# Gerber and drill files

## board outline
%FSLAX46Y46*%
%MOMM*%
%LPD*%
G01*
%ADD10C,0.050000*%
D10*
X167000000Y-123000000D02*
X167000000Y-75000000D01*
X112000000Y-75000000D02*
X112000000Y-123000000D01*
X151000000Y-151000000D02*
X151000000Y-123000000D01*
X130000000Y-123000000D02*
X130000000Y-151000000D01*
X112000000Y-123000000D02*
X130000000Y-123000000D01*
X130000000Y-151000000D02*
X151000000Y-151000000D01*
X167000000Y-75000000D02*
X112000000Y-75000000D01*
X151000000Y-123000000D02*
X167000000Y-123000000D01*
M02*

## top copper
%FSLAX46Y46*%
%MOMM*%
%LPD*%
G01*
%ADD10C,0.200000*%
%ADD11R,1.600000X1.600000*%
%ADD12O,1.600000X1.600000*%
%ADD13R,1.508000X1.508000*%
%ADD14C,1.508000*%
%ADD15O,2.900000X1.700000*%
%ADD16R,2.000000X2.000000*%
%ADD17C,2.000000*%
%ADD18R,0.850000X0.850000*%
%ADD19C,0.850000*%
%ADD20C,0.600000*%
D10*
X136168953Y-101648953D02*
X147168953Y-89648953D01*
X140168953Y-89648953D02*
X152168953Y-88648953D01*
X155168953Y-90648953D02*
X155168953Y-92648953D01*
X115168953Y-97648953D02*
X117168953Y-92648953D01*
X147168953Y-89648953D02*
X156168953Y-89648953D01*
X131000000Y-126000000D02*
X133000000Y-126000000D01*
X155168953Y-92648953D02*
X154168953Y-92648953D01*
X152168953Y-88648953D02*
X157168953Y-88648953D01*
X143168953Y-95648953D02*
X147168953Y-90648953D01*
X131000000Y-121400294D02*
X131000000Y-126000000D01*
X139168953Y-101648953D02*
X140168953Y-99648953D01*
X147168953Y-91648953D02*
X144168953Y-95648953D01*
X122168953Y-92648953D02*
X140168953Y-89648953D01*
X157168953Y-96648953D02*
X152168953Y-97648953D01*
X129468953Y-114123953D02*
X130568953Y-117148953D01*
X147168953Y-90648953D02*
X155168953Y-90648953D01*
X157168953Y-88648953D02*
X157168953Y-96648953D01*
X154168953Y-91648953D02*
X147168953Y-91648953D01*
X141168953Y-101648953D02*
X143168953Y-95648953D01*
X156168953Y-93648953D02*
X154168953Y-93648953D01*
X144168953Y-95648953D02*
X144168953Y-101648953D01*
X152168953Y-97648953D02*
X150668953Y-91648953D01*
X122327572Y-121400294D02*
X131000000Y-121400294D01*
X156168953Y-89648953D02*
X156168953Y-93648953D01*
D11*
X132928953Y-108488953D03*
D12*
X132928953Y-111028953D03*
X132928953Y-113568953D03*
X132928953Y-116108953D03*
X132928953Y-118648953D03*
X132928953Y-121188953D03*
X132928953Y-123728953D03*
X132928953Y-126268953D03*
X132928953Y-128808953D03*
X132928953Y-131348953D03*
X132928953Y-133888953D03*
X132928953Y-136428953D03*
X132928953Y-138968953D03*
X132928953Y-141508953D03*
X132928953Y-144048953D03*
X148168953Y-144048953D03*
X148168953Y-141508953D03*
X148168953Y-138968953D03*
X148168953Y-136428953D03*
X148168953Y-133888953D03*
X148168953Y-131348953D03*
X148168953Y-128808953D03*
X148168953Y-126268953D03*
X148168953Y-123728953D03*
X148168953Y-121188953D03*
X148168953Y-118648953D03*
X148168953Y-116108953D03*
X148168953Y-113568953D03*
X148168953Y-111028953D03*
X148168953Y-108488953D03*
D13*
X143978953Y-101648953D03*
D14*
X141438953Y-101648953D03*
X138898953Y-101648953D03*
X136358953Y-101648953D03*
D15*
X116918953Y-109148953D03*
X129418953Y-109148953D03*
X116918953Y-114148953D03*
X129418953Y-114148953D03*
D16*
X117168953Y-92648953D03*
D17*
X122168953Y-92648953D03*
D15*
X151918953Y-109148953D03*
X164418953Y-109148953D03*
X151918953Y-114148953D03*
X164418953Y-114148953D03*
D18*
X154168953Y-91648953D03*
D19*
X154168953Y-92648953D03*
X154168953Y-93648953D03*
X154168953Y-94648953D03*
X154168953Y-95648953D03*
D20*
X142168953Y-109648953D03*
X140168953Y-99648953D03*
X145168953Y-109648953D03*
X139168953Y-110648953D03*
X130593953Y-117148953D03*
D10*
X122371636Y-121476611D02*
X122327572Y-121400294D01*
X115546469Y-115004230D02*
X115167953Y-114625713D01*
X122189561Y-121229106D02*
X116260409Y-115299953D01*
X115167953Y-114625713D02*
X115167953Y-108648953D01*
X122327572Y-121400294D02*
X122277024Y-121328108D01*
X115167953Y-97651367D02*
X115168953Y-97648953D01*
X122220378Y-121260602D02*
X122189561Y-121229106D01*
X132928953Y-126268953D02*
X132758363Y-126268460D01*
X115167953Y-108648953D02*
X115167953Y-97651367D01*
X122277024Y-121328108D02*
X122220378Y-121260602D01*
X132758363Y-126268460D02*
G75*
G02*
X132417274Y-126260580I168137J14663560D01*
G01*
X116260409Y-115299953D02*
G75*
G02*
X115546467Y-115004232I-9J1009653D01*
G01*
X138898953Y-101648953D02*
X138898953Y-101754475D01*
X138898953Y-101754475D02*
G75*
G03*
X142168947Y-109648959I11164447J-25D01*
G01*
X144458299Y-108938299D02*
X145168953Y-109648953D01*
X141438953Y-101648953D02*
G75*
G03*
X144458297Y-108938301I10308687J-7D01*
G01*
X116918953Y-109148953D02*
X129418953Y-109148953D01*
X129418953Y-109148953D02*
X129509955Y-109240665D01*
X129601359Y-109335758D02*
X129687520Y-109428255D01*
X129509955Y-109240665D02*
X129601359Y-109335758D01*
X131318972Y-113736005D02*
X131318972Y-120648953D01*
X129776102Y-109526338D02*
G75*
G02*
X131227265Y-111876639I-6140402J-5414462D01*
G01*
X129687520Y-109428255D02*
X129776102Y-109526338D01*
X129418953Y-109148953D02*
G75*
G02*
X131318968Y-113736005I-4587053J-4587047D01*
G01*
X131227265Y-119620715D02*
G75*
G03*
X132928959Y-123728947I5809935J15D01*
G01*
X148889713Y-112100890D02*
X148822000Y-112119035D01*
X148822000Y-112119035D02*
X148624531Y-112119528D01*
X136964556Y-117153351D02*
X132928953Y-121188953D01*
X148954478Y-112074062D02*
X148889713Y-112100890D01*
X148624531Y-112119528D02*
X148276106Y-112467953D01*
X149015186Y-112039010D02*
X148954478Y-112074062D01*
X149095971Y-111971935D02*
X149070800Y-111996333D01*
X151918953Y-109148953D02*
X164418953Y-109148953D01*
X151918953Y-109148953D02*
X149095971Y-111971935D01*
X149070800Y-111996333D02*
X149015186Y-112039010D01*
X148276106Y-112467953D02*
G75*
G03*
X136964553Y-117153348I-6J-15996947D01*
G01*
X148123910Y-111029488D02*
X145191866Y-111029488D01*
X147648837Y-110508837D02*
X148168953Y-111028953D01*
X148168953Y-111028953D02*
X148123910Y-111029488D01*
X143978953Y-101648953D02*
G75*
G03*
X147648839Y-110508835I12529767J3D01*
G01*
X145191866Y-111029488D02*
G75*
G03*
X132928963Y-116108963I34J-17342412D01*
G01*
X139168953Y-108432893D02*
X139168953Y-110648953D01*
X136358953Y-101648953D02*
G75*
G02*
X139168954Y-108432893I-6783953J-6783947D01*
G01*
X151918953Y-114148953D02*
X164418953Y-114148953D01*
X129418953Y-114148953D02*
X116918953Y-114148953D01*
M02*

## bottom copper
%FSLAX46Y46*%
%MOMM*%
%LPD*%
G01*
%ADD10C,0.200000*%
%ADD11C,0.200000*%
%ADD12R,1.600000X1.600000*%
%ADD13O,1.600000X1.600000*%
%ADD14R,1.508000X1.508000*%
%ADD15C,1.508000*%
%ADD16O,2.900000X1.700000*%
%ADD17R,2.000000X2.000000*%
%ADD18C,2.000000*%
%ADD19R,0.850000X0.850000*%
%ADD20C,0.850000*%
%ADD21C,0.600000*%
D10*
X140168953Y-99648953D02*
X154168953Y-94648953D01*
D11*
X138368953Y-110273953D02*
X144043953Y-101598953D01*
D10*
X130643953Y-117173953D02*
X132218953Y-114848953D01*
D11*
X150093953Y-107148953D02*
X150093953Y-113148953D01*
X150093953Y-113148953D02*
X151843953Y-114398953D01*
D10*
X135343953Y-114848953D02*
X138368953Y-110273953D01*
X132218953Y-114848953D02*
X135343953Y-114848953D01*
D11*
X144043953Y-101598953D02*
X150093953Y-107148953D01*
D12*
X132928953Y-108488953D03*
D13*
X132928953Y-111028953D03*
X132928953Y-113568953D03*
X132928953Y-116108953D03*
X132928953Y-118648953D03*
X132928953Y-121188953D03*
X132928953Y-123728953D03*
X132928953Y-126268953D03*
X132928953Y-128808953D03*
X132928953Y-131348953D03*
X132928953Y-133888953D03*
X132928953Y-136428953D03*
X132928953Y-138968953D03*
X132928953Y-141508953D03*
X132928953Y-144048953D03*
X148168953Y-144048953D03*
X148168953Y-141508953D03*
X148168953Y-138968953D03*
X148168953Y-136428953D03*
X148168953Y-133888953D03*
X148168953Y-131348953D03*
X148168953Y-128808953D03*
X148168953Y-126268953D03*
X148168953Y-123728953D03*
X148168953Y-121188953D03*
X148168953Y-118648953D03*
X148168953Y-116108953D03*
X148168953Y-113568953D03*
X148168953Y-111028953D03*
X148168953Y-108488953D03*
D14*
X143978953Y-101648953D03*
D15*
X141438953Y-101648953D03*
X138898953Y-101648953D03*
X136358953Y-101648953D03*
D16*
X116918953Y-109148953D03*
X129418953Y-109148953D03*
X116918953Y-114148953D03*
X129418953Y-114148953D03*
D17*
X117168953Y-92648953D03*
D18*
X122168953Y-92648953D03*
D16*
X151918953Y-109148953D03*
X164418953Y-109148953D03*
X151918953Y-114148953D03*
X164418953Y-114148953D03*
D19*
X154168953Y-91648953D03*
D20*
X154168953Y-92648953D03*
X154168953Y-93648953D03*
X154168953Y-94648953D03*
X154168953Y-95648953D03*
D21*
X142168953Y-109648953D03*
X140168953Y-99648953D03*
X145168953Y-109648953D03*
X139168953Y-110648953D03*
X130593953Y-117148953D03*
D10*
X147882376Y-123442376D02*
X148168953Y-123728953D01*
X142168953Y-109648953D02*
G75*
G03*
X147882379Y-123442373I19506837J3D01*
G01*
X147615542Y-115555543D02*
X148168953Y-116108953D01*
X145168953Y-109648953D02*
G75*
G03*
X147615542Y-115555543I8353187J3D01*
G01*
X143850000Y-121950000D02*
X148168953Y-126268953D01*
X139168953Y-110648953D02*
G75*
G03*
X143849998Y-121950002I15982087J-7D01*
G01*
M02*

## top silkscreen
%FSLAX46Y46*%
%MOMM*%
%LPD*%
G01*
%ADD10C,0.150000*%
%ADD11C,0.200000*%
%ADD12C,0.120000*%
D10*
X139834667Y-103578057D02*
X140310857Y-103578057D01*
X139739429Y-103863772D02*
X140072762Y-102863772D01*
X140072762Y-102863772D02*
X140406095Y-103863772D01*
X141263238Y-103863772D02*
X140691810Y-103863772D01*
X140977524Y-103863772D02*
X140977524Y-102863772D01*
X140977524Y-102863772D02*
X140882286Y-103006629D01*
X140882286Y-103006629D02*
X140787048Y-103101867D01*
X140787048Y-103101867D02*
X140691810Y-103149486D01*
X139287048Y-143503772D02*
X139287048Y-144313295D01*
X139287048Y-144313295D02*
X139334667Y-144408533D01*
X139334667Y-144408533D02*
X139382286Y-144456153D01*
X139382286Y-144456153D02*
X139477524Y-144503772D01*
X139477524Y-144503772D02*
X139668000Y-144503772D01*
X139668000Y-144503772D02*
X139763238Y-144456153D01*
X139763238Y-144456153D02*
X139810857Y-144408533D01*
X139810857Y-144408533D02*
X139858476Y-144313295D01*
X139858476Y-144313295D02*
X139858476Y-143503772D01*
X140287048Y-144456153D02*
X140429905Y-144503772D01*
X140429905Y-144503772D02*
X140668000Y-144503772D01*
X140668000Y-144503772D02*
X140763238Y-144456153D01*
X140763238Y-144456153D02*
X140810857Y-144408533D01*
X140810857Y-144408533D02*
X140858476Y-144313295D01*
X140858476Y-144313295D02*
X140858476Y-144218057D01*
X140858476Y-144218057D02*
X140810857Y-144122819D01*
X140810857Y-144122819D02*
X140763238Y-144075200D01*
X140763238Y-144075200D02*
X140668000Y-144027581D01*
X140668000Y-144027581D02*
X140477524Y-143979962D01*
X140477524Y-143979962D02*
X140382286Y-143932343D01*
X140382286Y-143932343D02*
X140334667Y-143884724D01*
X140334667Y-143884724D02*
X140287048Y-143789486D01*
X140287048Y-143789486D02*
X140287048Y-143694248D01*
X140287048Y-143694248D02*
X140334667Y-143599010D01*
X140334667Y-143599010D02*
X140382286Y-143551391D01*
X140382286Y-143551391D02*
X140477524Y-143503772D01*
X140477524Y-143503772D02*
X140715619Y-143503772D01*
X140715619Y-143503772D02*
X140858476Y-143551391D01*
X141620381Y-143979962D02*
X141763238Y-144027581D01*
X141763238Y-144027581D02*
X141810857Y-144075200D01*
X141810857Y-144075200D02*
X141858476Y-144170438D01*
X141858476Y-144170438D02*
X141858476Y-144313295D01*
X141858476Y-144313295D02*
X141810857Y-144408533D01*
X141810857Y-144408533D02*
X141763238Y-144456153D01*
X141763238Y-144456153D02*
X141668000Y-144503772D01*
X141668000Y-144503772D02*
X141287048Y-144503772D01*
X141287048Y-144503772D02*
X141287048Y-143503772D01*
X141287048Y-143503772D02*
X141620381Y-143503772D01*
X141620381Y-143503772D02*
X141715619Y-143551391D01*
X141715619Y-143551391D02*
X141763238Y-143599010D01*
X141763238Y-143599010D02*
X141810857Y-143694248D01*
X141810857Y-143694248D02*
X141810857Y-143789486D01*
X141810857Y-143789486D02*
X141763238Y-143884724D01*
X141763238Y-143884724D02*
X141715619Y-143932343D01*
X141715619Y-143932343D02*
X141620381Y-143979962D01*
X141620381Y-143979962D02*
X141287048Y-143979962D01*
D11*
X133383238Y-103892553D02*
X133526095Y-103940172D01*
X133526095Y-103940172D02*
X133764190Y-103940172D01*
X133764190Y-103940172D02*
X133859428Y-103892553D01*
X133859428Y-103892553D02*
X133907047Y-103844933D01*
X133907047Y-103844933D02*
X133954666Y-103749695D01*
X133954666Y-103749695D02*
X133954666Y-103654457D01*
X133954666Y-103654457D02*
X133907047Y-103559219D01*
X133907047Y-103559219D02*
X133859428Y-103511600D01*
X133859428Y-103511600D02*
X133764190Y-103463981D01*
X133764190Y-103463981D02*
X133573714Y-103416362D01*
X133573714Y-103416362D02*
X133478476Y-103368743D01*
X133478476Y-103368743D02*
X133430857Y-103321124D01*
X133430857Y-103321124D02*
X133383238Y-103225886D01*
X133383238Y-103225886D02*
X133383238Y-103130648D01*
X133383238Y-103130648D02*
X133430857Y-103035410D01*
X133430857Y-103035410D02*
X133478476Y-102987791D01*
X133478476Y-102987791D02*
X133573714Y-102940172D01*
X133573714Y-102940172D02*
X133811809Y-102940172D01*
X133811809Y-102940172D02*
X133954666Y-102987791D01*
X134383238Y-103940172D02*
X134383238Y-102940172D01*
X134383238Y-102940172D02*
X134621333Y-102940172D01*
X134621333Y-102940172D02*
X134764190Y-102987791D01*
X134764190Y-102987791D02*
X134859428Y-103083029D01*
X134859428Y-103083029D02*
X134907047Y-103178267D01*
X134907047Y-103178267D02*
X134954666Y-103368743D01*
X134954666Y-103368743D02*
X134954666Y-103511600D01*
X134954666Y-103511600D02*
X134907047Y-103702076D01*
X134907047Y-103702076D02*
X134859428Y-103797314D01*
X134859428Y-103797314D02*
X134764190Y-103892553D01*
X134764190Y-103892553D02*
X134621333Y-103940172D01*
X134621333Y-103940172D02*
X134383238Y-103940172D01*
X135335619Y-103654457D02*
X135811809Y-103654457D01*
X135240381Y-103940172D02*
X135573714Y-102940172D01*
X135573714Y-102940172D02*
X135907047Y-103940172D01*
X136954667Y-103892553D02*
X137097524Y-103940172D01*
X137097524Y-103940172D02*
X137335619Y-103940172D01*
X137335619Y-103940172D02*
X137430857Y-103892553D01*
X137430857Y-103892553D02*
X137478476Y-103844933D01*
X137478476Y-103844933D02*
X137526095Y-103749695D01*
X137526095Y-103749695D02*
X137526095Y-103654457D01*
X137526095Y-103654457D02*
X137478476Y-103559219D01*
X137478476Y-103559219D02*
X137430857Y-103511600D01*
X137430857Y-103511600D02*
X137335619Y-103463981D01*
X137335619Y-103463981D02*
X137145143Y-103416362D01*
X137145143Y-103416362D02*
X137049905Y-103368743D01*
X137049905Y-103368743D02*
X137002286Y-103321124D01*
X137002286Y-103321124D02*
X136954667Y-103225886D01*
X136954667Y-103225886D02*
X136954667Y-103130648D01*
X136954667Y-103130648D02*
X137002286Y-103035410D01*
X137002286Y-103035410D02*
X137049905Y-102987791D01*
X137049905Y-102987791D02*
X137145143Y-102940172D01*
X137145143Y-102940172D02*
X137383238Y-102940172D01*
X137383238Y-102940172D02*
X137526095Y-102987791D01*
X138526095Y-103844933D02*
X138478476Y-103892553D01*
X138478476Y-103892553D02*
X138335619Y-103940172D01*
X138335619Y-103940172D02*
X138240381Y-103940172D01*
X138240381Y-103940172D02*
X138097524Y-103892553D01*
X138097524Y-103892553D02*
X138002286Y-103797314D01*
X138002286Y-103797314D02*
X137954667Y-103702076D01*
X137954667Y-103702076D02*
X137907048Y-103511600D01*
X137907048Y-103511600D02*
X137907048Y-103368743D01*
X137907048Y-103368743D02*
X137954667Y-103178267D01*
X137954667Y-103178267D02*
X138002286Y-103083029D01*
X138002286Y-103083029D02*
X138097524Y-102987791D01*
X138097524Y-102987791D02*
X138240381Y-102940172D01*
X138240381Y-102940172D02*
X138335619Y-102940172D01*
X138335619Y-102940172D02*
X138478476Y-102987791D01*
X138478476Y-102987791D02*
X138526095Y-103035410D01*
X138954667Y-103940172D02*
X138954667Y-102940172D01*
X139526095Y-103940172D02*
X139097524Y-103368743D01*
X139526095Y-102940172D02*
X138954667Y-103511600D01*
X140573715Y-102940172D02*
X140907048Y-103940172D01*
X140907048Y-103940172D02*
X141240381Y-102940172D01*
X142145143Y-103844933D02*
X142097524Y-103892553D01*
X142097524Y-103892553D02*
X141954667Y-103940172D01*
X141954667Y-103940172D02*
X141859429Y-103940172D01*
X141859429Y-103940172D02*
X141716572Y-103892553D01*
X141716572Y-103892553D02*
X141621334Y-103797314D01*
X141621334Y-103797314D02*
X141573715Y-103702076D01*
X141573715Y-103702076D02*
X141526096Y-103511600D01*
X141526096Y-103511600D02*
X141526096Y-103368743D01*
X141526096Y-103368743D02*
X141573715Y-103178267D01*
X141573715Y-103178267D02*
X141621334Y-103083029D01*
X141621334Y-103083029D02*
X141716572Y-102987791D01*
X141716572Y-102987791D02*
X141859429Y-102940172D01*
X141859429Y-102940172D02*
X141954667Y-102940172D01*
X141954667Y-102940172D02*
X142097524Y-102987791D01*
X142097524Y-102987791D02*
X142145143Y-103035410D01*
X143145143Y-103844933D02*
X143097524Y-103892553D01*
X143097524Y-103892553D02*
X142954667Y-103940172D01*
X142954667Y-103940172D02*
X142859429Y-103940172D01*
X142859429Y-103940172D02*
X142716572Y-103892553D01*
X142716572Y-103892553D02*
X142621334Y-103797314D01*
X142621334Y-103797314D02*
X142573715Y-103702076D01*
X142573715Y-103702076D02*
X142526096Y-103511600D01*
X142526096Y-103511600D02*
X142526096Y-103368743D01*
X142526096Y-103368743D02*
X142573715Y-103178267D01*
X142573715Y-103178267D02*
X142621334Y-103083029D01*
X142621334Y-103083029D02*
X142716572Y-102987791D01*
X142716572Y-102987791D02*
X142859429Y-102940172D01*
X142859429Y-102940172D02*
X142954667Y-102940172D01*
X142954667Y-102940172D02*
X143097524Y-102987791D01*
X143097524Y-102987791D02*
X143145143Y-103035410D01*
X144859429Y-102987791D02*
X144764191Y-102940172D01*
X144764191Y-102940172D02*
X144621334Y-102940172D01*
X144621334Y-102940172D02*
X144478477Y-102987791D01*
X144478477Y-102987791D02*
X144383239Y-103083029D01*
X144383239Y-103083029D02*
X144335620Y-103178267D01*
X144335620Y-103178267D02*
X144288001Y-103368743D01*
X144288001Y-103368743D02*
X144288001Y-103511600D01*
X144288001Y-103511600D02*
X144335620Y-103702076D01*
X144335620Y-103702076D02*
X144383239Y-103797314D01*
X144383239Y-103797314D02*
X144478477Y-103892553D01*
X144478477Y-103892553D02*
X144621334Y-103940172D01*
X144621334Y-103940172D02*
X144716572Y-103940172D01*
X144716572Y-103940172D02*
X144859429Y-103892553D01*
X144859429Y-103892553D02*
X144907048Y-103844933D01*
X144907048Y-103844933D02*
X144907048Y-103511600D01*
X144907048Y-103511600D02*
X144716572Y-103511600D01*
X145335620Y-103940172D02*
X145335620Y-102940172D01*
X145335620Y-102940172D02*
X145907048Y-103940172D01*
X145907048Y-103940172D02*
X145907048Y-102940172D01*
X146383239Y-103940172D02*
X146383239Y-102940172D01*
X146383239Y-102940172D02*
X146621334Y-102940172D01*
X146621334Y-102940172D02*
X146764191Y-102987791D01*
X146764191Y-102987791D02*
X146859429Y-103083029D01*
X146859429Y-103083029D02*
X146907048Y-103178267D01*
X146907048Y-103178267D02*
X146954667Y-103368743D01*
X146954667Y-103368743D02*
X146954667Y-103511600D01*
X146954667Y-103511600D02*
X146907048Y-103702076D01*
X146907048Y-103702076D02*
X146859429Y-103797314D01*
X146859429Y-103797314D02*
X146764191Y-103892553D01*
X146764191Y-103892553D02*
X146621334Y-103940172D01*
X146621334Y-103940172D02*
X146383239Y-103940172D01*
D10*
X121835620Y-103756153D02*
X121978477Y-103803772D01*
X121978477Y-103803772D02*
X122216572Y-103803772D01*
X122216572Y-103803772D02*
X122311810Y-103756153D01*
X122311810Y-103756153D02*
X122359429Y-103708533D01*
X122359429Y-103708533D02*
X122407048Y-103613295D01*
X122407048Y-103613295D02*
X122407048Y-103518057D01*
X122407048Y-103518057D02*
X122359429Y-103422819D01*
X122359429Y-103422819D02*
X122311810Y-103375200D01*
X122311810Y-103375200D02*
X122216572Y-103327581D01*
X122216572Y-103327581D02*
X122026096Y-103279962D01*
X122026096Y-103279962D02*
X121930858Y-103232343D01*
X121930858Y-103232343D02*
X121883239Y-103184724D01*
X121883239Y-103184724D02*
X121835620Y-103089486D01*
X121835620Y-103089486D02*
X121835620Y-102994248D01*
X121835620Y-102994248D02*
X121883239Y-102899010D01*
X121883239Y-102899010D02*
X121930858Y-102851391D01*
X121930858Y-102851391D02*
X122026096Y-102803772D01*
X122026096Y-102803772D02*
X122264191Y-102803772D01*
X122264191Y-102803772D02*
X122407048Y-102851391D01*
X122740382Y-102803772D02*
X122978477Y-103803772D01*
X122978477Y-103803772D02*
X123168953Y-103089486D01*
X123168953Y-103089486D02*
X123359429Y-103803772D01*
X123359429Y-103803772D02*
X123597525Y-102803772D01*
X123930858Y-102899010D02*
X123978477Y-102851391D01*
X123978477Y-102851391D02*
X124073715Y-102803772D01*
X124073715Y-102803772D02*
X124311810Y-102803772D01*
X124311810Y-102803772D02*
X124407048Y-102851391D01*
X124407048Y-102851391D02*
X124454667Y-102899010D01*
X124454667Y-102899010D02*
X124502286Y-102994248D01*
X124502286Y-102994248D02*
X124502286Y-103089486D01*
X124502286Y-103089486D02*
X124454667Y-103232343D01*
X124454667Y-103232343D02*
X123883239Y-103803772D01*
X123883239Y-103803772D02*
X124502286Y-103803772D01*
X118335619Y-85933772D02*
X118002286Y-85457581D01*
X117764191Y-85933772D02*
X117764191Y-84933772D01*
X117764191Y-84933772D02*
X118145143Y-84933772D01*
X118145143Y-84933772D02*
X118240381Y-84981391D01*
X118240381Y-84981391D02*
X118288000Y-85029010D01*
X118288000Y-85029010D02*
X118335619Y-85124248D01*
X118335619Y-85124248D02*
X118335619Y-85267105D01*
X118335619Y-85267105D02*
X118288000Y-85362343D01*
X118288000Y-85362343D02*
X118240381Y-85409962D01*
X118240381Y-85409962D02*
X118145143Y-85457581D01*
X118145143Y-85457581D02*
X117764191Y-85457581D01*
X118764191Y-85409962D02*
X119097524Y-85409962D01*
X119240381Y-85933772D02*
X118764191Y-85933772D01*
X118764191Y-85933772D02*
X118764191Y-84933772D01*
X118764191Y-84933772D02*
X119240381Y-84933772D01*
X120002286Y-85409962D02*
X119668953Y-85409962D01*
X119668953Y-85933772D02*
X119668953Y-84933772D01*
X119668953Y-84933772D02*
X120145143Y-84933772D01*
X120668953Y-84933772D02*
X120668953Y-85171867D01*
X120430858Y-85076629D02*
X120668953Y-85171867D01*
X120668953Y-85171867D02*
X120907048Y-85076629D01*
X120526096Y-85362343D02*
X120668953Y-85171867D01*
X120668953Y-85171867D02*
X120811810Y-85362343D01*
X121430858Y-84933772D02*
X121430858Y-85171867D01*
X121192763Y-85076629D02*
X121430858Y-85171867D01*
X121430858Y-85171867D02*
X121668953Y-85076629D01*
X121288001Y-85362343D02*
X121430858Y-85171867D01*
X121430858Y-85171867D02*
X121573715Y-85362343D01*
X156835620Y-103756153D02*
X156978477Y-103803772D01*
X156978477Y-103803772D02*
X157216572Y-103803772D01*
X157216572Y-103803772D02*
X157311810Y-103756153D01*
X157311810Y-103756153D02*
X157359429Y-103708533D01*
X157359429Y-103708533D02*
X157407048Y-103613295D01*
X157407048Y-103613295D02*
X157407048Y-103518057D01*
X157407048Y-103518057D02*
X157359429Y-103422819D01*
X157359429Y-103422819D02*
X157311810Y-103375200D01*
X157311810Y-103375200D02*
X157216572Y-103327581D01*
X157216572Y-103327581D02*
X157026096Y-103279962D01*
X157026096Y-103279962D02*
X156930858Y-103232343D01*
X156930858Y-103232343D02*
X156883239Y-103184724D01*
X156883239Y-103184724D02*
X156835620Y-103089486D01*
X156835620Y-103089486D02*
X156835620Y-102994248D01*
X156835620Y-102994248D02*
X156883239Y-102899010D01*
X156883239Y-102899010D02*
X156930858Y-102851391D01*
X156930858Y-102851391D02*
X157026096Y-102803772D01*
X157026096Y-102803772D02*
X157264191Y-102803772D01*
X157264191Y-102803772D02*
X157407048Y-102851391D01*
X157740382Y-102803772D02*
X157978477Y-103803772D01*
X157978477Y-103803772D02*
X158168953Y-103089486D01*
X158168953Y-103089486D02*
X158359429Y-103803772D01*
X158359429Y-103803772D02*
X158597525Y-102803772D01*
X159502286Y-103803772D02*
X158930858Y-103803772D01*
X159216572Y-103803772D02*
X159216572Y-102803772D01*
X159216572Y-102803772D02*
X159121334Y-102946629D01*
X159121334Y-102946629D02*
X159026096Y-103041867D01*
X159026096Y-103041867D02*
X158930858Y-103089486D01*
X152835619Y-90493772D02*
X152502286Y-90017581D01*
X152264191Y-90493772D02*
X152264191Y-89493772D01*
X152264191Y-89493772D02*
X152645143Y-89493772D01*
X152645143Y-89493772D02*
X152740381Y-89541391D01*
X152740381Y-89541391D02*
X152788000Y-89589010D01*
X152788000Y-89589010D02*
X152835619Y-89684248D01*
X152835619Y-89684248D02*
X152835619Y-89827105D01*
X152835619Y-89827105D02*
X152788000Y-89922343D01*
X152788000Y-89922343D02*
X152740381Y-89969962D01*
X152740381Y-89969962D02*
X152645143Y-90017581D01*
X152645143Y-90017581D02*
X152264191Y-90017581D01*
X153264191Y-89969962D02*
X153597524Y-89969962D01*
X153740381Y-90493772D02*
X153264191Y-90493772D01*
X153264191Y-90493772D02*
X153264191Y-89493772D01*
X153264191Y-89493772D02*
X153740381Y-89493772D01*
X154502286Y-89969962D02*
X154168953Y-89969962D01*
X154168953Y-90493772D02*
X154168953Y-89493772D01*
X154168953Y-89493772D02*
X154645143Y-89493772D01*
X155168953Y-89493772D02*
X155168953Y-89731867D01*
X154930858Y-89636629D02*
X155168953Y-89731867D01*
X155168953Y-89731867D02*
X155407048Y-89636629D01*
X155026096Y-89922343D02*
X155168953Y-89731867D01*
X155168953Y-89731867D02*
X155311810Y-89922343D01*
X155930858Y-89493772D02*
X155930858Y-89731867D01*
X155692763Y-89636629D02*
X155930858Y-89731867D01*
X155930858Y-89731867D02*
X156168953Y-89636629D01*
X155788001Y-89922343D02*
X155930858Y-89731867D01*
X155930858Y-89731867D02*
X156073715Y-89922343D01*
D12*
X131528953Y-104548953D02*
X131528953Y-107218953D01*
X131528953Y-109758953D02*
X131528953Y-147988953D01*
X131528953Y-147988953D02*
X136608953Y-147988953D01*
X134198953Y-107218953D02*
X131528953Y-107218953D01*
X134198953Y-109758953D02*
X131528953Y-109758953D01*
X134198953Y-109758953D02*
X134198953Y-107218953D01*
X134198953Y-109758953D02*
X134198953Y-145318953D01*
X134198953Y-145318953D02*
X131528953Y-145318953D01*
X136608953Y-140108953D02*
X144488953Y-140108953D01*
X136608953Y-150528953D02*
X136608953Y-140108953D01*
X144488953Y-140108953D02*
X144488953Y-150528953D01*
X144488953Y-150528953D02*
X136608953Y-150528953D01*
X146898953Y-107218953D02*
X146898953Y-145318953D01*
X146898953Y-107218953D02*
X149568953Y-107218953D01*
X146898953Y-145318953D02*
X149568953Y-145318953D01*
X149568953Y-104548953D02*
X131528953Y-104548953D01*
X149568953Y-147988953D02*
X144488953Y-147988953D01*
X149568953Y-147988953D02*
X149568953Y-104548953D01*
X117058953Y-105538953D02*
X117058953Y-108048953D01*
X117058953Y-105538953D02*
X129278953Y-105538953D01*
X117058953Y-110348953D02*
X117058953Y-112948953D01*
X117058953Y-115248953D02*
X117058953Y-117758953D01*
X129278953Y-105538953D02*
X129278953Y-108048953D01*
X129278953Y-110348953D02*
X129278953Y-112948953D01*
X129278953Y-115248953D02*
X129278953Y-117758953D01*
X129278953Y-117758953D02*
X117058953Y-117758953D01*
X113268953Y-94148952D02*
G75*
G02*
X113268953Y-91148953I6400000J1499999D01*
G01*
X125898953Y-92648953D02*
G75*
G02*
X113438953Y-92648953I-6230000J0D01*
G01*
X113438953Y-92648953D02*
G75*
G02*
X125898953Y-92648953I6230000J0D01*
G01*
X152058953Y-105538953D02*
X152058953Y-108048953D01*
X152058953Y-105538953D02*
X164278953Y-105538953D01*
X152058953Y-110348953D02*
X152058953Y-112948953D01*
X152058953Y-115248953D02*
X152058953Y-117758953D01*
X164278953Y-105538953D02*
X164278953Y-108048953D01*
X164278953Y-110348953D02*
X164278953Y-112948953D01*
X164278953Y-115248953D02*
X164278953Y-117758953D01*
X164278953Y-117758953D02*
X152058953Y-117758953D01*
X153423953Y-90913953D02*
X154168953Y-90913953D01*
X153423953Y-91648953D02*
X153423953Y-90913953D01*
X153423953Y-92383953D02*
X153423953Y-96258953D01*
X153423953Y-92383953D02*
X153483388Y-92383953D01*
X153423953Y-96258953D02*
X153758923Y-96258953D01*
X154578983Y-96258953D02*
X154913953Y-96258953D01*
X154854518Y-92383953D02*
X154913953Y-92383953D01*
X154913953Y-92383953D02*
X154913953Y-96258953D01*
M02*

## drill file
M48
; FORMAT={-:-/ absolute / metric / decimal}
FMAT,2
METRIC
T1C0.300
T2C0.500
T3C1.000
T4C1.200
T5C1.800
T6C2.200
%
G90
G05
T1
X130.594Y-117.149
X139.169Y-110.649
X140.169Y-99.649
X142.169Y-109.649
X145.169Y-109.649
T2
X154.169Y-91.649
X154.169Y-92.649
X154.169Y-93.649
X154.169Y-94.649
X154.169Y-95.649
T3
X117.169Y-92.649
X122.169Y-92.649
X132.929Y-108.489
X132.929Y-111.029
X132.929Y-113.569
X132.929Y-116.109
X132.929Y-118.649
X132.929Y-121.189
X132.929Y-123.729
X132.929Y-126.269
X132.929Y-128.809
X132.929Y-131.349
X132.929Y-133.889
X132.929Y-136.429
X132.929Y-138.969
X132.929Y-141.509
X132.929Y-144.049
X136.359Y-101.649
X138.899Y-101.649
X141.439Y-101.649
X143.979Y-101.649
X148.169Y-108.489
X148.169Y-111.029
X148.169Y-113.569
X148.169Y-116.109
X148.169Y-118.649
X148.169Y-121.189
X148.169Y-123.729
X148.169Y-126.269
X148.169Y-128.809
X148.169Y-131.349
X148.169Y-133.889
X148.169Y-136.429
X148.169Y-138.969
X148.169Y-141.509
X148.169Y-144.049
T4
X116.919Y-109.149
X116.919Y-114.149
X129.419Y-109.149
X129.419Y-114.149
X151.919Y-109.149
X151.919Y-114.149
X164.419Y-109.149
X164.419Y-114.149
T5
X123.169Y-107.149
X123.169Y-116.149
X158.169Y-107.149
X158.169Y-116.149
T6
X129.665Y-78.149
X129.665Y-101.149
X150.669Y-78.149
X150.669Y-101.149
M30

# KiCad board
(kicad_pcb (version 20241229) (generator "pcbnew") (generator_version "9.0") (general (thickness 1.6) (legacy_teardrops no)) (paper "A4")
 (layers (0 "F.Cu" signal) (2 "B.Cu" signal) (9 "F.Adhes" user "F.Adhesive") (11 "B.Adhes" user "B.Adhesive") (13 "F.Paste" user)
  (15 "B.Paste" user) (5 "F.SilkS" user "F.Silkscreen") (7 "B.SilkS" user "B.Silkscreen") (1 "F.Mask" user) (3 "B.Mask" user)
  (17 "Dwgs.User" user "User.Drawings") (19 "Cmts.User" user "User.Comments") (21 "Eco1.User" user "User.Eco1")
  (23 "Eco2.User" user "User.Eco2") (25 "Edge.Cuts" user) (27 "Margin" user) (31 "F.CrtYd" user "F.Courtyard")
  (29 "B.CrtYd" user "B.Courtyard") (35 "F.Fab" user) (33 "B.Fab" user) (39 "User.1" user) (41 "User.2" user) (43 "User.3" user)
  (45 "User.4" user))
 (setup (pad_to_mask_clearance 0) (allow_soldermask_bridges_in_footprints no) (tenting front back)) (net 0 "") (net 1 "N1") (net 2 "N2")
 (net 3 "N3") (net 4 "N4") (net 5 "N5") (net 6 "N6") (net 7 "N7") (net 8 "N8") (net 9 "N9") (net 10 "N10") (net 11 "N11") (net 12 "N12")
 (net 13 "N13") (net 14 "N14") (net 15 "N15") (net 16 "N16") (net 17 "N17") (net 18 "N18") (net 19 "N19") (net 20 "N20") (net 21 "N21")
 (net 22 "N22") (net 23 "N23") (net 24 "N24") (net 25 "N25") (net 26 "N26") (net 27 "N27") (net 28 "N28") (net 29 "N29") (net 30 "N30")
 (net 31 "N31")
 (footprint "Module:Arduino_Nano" (layer "F.Cu") (at 132.928953 108.488953)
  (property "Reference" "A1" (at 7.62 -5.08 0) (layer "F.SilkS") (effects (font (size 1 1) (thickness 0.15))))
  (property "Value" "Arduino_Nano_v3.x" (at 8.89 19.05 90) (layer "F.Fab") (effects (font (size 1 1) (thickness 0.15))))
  (fp_line (start -1.4 -3.94) (end -1.4 -1.27) (stroke (width 0.12) (type solid)) (layer "F.SilkS"))
  (fp_line (start -1.4 1.27) (end -1.4 39.5) (stroke (width 0.12) (type solid)) (layer "F.SilkS"))
  (fp_line (start -1.4 39.5) (end 3.68 39.5) (stroke (width 0.12) (type solid)) (layer "F.SilkS"))
  (fp_line (start 1.27 -1.27) (end -1.4 -1.27) (stroke (width 0.12) (type solid)) (layer "F.SilkS"))
  (fp_line (start 1.27 1.27) (end -1.4 1.27) (stroke (width 0.12) (type solid)) (layer "F.SilkS"))
  (fp_line (start 1.27 1.27) (end 1.27 -1.27) (stroke (width 0.12) (type solid)) (layer "F.SilkS"))
  (fp_line (start 1.27 1.27) (end 1.27 36.83) (stroke (width 0.12) (type solid)) (layer "F.SilkS"))
  (fp_line (start 1.27 36.83) (end -1.4 36.83) (stroke (width 0.12) (type solid)) (layer "F.SilkS"))
  (fp_line (start 3.68 31.62) (end 11.56 31.62) (stroke (width 0.12) (type solid)) (layer "F.SilkS"))
  (fp_line (start 3.68 42.04) (end 3.68 31.62) (stroke (width 0.12) (type solid)) (layer "F.SilkS"))
  (fp_line (start 11.56 31.62) (end 11.56 42.04) (stroke (width 0.12) (type solid)) (layer "F.SilkS"))
  (fp_line (start 11.56 42.04) (end 3.68 42.04) (stroke (width 0.12) (type solid)) (layer "F.SilkS"))
  (fp_line (start 13.97 -1.27) (end 13.97 36.83) (stroke (width 0.12) (type solid)) (layer "F.SilkS"))
  (fp_line (start 13.97 -1.27) (end 16.64 -1.27) (stroke (width 0.12) (type solid)) (layer "F.SilkS"))
  (fp_line (start 13.97 36.83) (end 16.64 36.83) (stroke (width 0.12) (type solid)) (layer "F.SilkS"))
  (fp_line (start 16.64 -3.94) (end -1.4 -3.94) (stroke (width 0.12) (type solid)) (layer "F.SilkS"))
  (fp_line (start 16.64 39.5) (end 11.56 39.5) (stroke (width 0.12) (type solid)) (layer "F.SilkS"))
  (fp_line (start 16.64 39.5) (end 16.64 -3.94) (stroke (width 0.12) (type solid)) (layer "F.SilkS"))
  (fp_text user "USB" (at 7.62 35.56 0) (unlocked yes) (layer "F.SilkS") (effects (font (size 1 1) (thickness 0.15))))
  (pad "1" thru_hole rect (at 0 0) (size 1.6 1.6) (drill 1) (layers "*.Cu" "*.Mask") (remove_unused_layers no) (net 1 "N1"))
  (pad "2" thru_hole oval (at 0 2.54) (size 1.6 1.6) (drill 1) (layers "*.Cu" "*.Mask") (remove_unused_layers no) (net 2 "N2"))
  (pad "3" thru_hole oval (at 0 5.08) (size 1.6 1.6) (drill 1) (layers "*.Cu" "*.Mask") (remove_unused_layers no) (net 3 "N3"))
  (pad "4" thru_hole oval (at 0 7.62) (size 1.6 1.6) (drill 1) (layers "*.Cu" "*.Mask") (remove_unused_layers no) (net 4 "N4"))
  (pad "5" thru_hole oval (at 0 10.16) (size 1.6 1.6) (drill 1) (layers "*.Cu" "*.Mask") (remove_unused_layers no) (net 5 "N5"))
  (pad "6" thru_hole oval (at 0 12.7) (size 1.6 1.6) (drill 1) (layers "*.Cu" "*.Mask") (remove_unused_layers no) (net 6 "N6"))
  (pad "7" thru_hole oval (at 0 15.24) (size 1.6 1.6) (drill 1) (layers "*.Cu" "*.Mask") (remove_unused_layers no) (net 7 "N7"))
  (pad "8" thru_hole oval (at 0 17.78) (size 1.6 1.6) (drill 1) (layers "*.Cu" "*.Mask") (remove_unused_layers no) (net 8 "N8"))
  (pad "9" thru_hole oval (at 0 20.32) (size 1.6 1.6) (drill 1) (layers "*.Cu" "*.Mask") (remove_unused_layers no) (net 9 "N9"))
  (pad "10" thru_hole oval (at 0 22.86) (size 1.6 1.6) (drill 1) (layers "*.Cu" "*.Mask") (remove_unused_layers no) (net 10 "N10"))
  (pad "11" thru_hole oval (at 0 25.4) (size 1.6 1.6) (drill 1) (layers "*.Cu" "*.Mask") (remove_unused_layers no) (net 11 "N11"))
  (pad "12" thru_hole oval (at 0 27.94) (size 1.6 1.6) (drill 1) (layers "*.Cu" "*.Mask") (remove_unused_layers no) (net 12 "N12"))
  (pad "13" thru_hole oval (at 0 30.48) (size 1.6 1.6) (drill 1) (layers "*.Cu" "*.Mask") (remove_unused_layers no) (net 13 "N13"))
  (pad "14" thru_hole oval (at 0 33.02) (size 1.6 1.6) (drill 1) (layers "*.Cu" "*.Mask") (remove_unused_layers no) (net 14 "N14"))
  (pad "15" thru_hole oval (at 0 35.56) (size 1.6 1.6) (drill 1) (layers "*.Cu" "*.Mask") (remove_unused_layers no) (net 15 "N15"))
  (pad "16" thru_hole oval (at 15.24 35.56) (size 1.6 1.6) (drill 1) (layers "*.Cu" "*.Mask") (remove_unused_layers no) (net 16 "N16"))
  (pad "17" thru_hole oval (at 15.24 33.02) (size 1.6 1.6) (drill 1) (layers "*.Cu" "*.Mask") (remove_unused_layers no) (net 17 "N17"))
  (pad "18" thru_hole oval (at 15.24 30.48) (size 1.6 1.6) (drill 1) (layers "*.Cu" "*.Mask") (remove_unused_layers no) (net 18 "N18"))
  (pad "19" thru_hole oval (at 15.24 27.94) (size 1.6 1.6) (drill 1) (layers "*.Cu" "*.Mask") (remove_unused_layers no) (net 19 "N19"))
  (pad "20" thru_hole oval (at 15.24 25.4) (size 1.6 1.6) (drill 1) (layers "*.Cu" "*.Mask") (remove_unused_layers no) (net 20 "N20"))
  (pad "21" thru_hole oval (at 15.24 22.86) (size 1.6 1.6) (drill 1) (layers "*.Cu" "*.Mask") (remove_unused_layers no) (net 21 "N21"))
  (pad "22" thru_hole oval (at 15.24 20.32) (size 1.6 1.6) (drill 1) (layers "*.Cu" "*.Mask") (remove_unused_layers no) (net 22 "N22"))
  (pad "23" thru_hole oval (at 15.24 17.78) (size 1.6 1.6) (drill 1) (layers "*.Cu" "*.Mask") (remove_unused_layers no) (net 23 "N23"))
  (pad "24" thru_hole oval (at 15.24 15.24) (size 1.6 1.6) (drill 1) (layers "*.Cu" "*.Mask") (remove_unused_layers no) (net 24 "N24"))
  (pad "25" thru_hole oval (at 15.24 12.7) (size 1.6 1.6) (drill 1) (layers "*.Cu" "*.Mask") (remove_unused_layers no) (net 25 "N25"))
  (pad "26" thru_hole oval (at 15.24 10.16) (size 1.6 1.6) (drill 1) (layers "*.Cu" "*.Mask") (remove_unused_layers no) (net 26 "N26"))
  (pad "27" thru_hole oval (at 15.24 7.62) (size 1.6 1.6) (drill 1) (layers "*.Cu" "*.Mask") (remove_unused_layers no) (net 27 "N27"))
  (pad "28" thru_hole oval (at 15.24 5.08) (size 1.6 1.6) (drill 1) (layers "*.Cu" "*.Mask") (remove_unused_layers no) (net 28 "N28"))
  (pad "29" thru_hole oval (at 15.24 2.54) (size 1.6 1.6) (drill 1) (layers "*.Cu" "*.Mask") (remove_unused_layers no) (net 4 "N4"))
  (pad "30" thru_hole oval (at 15.24 0) (size 1.6 1.6) (drill 1) (layers "*.Cu" "*.Mask") (remove_unused_layers no) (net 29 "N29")))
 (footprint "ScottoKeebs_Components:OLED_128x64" (layer "F.Cu") (at 140.168953 89.648953)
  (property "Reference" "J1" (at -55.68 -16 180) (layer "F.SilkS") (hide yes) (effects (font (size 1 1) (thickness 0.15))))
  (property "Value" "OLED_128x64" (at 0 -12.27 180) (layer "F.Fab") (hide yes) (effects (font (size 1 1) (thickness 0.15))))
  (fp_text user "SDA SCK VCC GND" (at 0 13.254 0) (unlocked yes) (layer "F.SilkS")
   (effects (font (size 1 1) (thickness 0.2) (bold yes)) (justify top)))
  (pad "" np_thru_hole circle (at -10.50445 -11.5 180) (size 2.2 2.2) (drill 2.2) (layers "*.Cu" "*.Mask") (solder_mask_margin 0.102))
  (pad "" np_thru_hole circle (at -10.50445 11.5 180) (size 2.2 2.2) (drill 2.2) (layers "*.Cu" "*.Mask") (solder_mask_margin 0.102))
  (pad "" np_thru_hole circle (at 10.5 -11.5 180) (size 2.2 2.2) (drill 2.2) (layers "*.Cu" "*.Mask") (solder_mask_margin 0.102))
  (pad "" np_thru_hole circle (at 10.5 11.5 180) (size 2.2 2.2) (drill 2.2) (layers "*.Cu" "*.Mask") (solder_mask_margin 0.102))
  (pad "1" thru_hole rect (at 3.81 12 180) (size 1.508 1.508) (drill 1) (layers "*.Cu" "*.Mask") (remove_unused_layers no) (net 4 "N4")
   (solder_mask_margin 0.102))
  (pad "2" thru_hole circle (at 1.27 12 180) (size 1.508 1.508) (drill 1) (layers "*.Cu" "*.Mask") (remove_unused_layers no) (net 27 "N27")
   (solder_mask_margin 0.102))
  (pad "3" thru_hole circle (at -1.27 12 180) (size 1.508 1.508) (drill 1) (layers "*.Cu" "*.Mask") (remove_unused_layers no) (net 24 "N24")
   (solder_mask_margin 0.102))
  (pad "4" thru_hole circle (at -3.81 12 180) (size 1.508 1.508) (drill 1) (layers "*.Cu" "*.Mask") (remove_unused_layers no) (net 23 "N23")
   (solder_mask_margin 0.102)))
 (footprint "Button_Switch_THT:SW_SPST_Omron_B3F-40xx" (layer "F.Cu") (at 116.918953 109.148953)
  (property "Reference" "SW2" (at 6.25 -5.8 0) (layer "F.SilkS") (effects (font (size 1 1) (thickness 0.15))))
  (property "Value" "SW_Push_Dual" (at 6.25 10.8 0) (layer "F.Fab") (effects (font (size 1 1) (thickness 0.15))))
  (fp_line (start 0.14 -3.61) (end 0.14 -1.1) (stroke (width 0.12) (type default)) (layer "F.SilkS"))
  (fp_line (start 0.14 -3.61) (end 12.36 -3.61) (stroke (width 0.12) (type default)) (layer "F.SilkS"))
  (fp_line (start 0.14 1.2) (end 0.14 3.8) (stroke (width 0.12) (type default)) (layer "F.SilkS"))
  (fp_line (start 0.14 6.1) (end 0.14 8.61) (stroke (width 0.12) (type default)) (layer "F.SilkS"))
  (fp_line (start 12.36 -3.61) (end 12.36 -1.1) (stroke (width 0.12) (type default)) (layer "F.SilkS"))
  (fp_line (start 12.36 1.2) (end 12.36 3.8) (stroke (width 0.12) (type default)) (layer "F.SilkS"))
  (fp_line (start 12.36 6.1) (end 12.36 8.61) (stroke (width 0.12) (type default)) (layer "F.SilkS"))
  (fp_line (start 12.36 8.61) (end 0.14 8.61) (stroke (width 0.12) (type default)) (layer "F.SilkS"))
  (pad "" np_thru_hole circle (at 6.25 -2) (size 1.8 1.8) (drill 1.8) (layers "*.Cu" "*.Mask"))
  (pad "" np_thru_hole circle (at 6.25 7) (size 1.8 1.8) (drill 1.8) (layers "*.Cu" "*.Mask"))
  (pad "1" thru_hole oval (at 0 0) (size 2.9 1.7) (drill 1.2) (layers "*.Cu" "*.Mask") (remove_unused_layers no) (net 7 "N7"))
  (pad "1" thru_hole oval (at 12.5 0) (size 2.9 1.7) (drill 1.2) (layers "*.Cu" "*.Mask") (remove_unused_layers no) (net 7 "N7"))
  (pad "2" thru_hole oval (at 0 5) (size 2.9 1.7) (drill 1.2) (layers "*.Cu" "*.Mask") (remove_unused_layers no) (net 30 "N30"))
  (pad "2" thru_hole oval (at 12.5 5) (size 2.9 1.7) (drill 1.2) (layers "*.Cu" "*.Mask") (remove_unused_layers no) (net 30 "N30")))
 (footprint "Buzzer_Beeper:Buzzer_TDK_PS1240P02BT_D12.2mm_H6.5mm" (layer "F.Cu") (at 117.168953 92.648953)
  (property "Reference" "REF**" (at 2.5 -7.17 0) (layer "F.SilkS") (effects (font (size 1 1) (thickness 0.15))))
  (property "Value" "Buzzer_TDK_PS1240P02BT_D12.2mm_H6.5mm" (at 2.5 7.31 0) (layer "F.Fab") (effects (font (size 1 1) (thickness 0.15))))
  (fp_arc (start -3.9 1.499999) (mid -4.073431 0) (end -3.9 -1.5) (stroke (width 0.12) (type solid)) (layer "F.SilkS"))
  (fp_circle (center 2.5 0) (end 8.73 0) (stroke (width 0.12) (type solid)) (fill no) (layer "F.SilkS"))
  (pad "1" thru_hole rect (at 0 0) (size 2 2) (drill 1) (layers "*.Cu" "*.Mask") (remove_unused_layers no))
  (pad "2" thru_hole circle (at 5 0) (size 2 2) (drill 1) (layers "*.Cu" "*.Mask") (remove_unused_layers no)))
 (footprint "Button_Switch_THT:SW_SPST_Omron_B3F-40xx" (layer "F.Cu") (at 151.918953 109.148953)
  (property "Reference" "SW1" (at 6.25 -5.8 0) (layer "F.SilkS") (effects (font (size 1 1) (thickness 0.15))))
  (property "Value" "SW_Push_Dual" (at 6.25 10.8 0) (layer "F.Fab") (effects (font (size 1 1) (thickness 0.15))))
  (fp_line (start 0.14 -3.61) (end 0.14 -1.1) (stroke (width 0.12) (type default)) (layer "F.SilkS"))
  (fp_line (start 0.14 -3.61) (end 12.36 -3.61) (stroke (width 0.12) (type default)) (layer "F.SilkS"))
  (fp_line (start 0.14 1.2) (end 0.14 3.8) (stroke (width 0.12) (type default)) (layer "F.SilkS"))
  (fp_line (start 0.14 6.1) (end 0.14 8.61) (stroke (width 0.12) (type default)) (layer "F.SilkS"))
  (fp_line (start 12.36 -3.61) (end 12.36 -1.1) (stroke (width 0.12) (type default)) (layer "F.SilkS"))
  (fp_line (start 12.36 1.2) (end 12.36 3.8) (stroke (width 0.12) (type default)) (layer "F.SilkS"))
  (fp_line (start 12.36 6.1) (end 12.36 8.61) (stroke (width 0.12) (type default)) (layer "F.SilkS"))
  (fp_line (start 12.36 8.61) (end 0.14 8.61) (stroke (width 0.12) (type default)) (layer "F.SilkS"))
  (pad "" np_thru_hole circle (at 6.25 -2) (size 1.8 1.8) (drill 1.8) (layers "*.Cu" "*.Mask"))
  (pad "" np_thru_hole circle (at 6.25 7) (size 1.8 1.8) (drill 1.8) (layers "*.Cu" "*.Mask"))
  (pad "1" thru_hole oval (at 0 0) (size 2.9 1.7) (drill 1.2) (layers "*.Cu" "*.Mask") (remove_unused_layers no) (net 6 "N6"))
  (pad "1" thru_hole oval (at 12.5 0) (size 2.9 1.7) (drill 1.2) (layers "*.Cu" "*.Mask") (remove_unused_layers no) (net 6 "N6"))
  (pad "2" thru_hole oval (at 0 5) (size 2.9 1.7) (drill 1.2) (layers "*.Cu" "*.Mask") (remove_unused_layers no) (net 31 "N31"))
  (pad "2" thru_hole oval (at 12.5 5) (size 2.9 1.7) (drill 1.2) (layers "*.Cu" "*.Mask") (remove_unused_layers no) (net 31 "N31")))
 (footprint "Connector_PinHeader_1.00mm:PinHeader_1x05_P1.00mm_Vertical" (layer "F.Cu") (at 154.168953 91.648953)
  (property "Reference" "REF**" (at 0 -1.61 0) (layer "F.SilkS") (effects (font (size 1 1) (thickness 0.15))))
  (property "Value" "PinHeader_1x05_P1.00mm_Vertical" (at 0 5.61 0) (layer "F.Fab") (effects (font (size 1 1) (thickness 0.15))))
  (fp_line (start -0.745 -0.735) (end 0 -0.735) (stroke (width 0.12) (type solid)) (layer "F.SilkS"))
  (fp_line (start -0.745 0) (end -0.745 -0.735) (stroke (width 0.12) (type solid)) (layer "F.SilkS"))
  (fp_line (start -0.745 0.735) (end -0.745 4.61) (stroke (width 0.12) (type solid)) (layer "F.SilkS"))
  (fp_line (start -0.745 0.735) (end -0.685565 0.735) (stroke (width 0.12) (type solid)) (layer "F.SilkS"))
  (fp_line (start -0.745 4.61) (end -0.41003 4.61) (stroke (width 0.12) (type solid)) (layer "F.SilkS"))
  (fp_line (start 0.41003 4.61) (end 0.745 4.61) (stroke (width 0.12) (type solid)) (layer "F.SilkS"))
  (fp_line (start 0.685565 0.735) (end 0.745 0.735) (stroke (width 0.12) (type solid)) (layer "F.SilkS"))
  (fp_line (start 0.745 0.735) (end 0.745 4.61) (stroke (width 0.12) (type solid)) (layer "F.SilkS"))
  (pad "1" thru_hole rect (at 0 0) (size 0.85 0.85) (drill 0.5) (layers "*.Cu" "*.Mask") (remove_unused_layers no))
  (pad "2" thru_hole circle (at 0 1) (size 0.85 0.85) (drill 0.5) (layers "*.Cu" "*.Mask") (remove_unused_layers no))
  (pad "3" thru_hole circle (at 0 2) (size 0.85 0.85) (drill 0.5) (layers "*.Cu" "*.Mask") (remove_unused_layers no))
  (pad "4" thru_hole circle (at 0 3) (size 0.85 0.85) (drill 0.5) (layers "*.Cu" "*.Mask") (remove_unused_layers no))
  (pad "5" thru_hole circle (at 0 4) (size 0.85 0.85) (drill 0.5) (layers "*.Cu" "*.Mask") (remove_unused_layers no)))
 (gr_line (start 136.168953 101.648953) (end 147.168953 89.648953) (stroke (width 0.2) (type default)) (layer "F.Cu") (net 23))
 (gr_line (start 140.168953 89.648953) (end 152.168953 88.648953) (stroke (width 0.2) (type default)) (layer "F.Cu") (net 4))
 (gr_line (start 155.168953 90.648953) (end 155.168953 92.648953) (stroke (width 0.2) (type default)) (layer "F.Cu") (net 27))
 (gr_line (start 115.168953 97.648953) (end 117.168953 92.648953) (stroke (width 0.2) (type default)) (layer "F.Cu") (net 8))
 (gr_line (start 147.168953 89.648953) (end 156.168953 89.648953) (stroke (width 0.2) (type default)) (layer "F.Cu") (net 23))
 (gr_line (start 131 126) (end 133 126) (stroke (width 0.2) (type default)) (layer "F.Cu") (net 8))
 (gr_line (start 155.168953 92.648953) (end 154.168953 92.648953) (stroke (width 0.2) (type default)) (layer "F.Cu") (net 27))
 (gr_line (start 152.168953 88.648953) (end 157.168953 88.648953) (stroke (width 0.2) (type default)) (layer "F.Cu") (net 4))
 (gr_line (start 143.168953 95.648953) (end 147.168953 90.648953) (stroke (width 0.2) (type default)) (layer "F.Cu") (net 27))
 (gr_line (start 131 121.400294) (end 131 126) (stroke (width 0.2) (type default)) (layer "F.Cu") (net 8))
 (gr_line (start 139.168953 101.648953) (end 140.168953 99.648953) (stroke (width 0.2) (type default)) (layer "F.Cu") (net 24))
 (gr_line (start 147.168953 91.648953) (end 144.168953 95.648953) (stroke (width 0.2) (type default)) (layer "F.Cu") (net 4))
 (gr_line (start 122.168953 92.648953) (end 140.168953 89.648953) (stroke (width 0.2) (type default)) (layer "F.Cu") (net 4))
 (gr_line (start 157.168953 96.648953) (end 152.168953 97.648953) (stroke (width 0.2) (type default)) (layer "F.Cu") (net 4))
 (gr_line (start 129.468953 114.123953) (end 130.568953 117.148953) (stroke (width 0.2) (type default)) (layer "F.Cu") (net 30))
 (gr_line (start 147.168953 90.648953) (end 155.168953 90.648953) (stroke (width 0.2) (type default)) (layer "F.Cu") (net 27))
 (gr_line (start 157.168953 88.648953) (end 157.168953 96.648953) (stroke (width 0.2) (type default)) (layer "F.Cu") (net 4))
 (gr_line (start 154.168953 91.648953) (end 147.168953 91.648953) (stroke (width 0.2) (type default)) (layer "F.Cu") (net 4))
 (gr_line (start 141.168953 101.648953) (end 143.168953 95.648953) (stroke (width 0.2) (type default)) (layer "F.Cu") (net 27))
 (gr_line (start 156.168953 93.648953) (end 154.168953 93.648953) (stroke (width 0.2) (type default)) (layer "F.Cu") (net 23))
 (gr_line (start 144.168953 95.648953) (end 144.168953 101.648953) (stroke (width 0.2) (type default)) (layer "F.Cu") (net 4))
 (gr_line (start 152.168953 97.648953) (end 150.668953 91.648953) (stroke (width 0.2) (type default)) (layer "F.Cu") (net 4))
 (gr_line (start 122.327572 121.400294) (end 131 121.400294) (stroke (width 0.2) (type default)) (layer "F.Cu") (net 8))
 (gr_line (start 156.168953 89.648953) (end 156.168953 93.648953) (stroke (width 0.2) (type default)) (layer "F.Cu") (net 23))
 (gr_line (start 140.168953 99.648953) (end 154.168953 94.648953) (stroke (width 0.2) (type default)) (layer "B.Cu") (net 24))
 (gr_line (start 138.368953 110.273953) (end 144.043953 101.598953) (stroke (width 0.2) (type default)) (layer "B.Cu"))
 (gr_line (start 130.643953 117.173953) (end 132.218953 114.848953) (stroke (width 0.2) (type default)) (layer "B.Cu") (net 30))
 (gr_line (start 150.093953 107.148953) (end 150.093953 113.148953) (stroke (width 0.2) (type default)) (layer "B.Cu"))
 (gr_line (start 150.093953 113.148953) (end 151.843953 114.398953) (stroke (width 0.2) (type default)) (layer "B.Cu"))
 (gr_line (start 135.343953 114.848953) (end 138.368953 110.273953) (stroke (width 0.2) (type default)) (layer "B.Cu") (net 30))
 (gr_line (start 132.218953 114.848953) (end 135.343953 114.848953) (stroke (width 0.2) (type default)) (layer "B.Cu") (net 30))
 (gr_line (start 144.043953 101.598953) (end 150.093953 107.148953) (stroke (width 0.2) (type default)) (layer "B.Cu"))
 (gr_line (start 167 123) (end 167 75) (stroke (width 0.05) (type default)) (layer "Edge.Cuts"))
 (gr_line (start 112 75) (end 112 123) (stroke (width 0.05) (type default)) (layer "Edge.Cuts"))
 (gr_line (start 151 151) (end 151 123) (stroke (width 0.05) (type default)) (layer "Edge.Cuts"))
 (gr_line (start 130 123) (end 130 151) (stroke (width 0.05) (type default)) (layer "Edge.Cuts"))
 (gr_line (start 112 123) (end 130 123) (stroke (width 0.05) (type default)) (layer "Edge.Cuts"))
 (gr_line (start 130 151) (end 151 151) (stroke (width 0.05) (type default)) (layer "Edge.Cuts"))
 (gr_line (start 167 75) (end 112 75) (stroke (width 0.05) (type default)) (layer "Edge.Cuts"))
 (gr_line (start 151 123) (end 167 123) (stroke (width 0.05) (type default)) (layer "Edge.Cuts"))
 (segment (start 122.371636 121.476611) (end 122.327572 121.400294) (width 0.2) (layer "F.Cu") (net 8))
 (segment (start 115.546469 115.00423) (end 115.167953 114.625713) (width 0.2) (layer "F.Cu") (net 8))
 (segment (start 122.189561 121.229106) (end 116.260409 115.299953) (width 0.2) (layer "F.Cu") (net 8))
 (segment (start 115.167953 114.625713) (end 115.167953 108.648953) (width 0.2) (layer "F.Cu") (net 8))
 (segment (start 122.327572 121.400294) (end 122.277024 121.328108) (width 0.2) (layer "F.Cu") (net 8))
 (segment (start 115.167953 97.651367) (end 115.168953 97.648953) (width 0.2) (layer "F.Cu") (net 8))
 (segment (start 122.220378 121.260602) (end 122.189561 121.229106) (width 0.2) (layer "F.Cu") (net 8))
 (segment (start 132.928953 126.268953) (end 132.758363 126.26846) (width 0.2) (layer "F.Cu") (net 8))
 (segment (start 115.167953 108.648953) (end 115.167953 97.651367) (width 0.2) (layer "F.Cu") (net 8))
 (segment (start 122.277024 121.328108) (end 122.220378 121.260602) (width 0.2) (layer "F.Cu") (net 8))
 (arc (start 132.758363 126.26846) (mid 132.587796 126.265512) (end 132.417274 126.26058) (width 0.2) (layer "F.Cu") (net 8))
 (arc (start 116.260409 115.299953) (mid 115.874028 115.223097) (end 115.546469 115.00423) (width 0.2) (layer "F.Cu") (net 8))
 (segment (start 138.898953 101.648953) (end 138.898953 101.754475) (width 0.2) (layer "F.Cu") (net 24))
 (via (at 142.168953 109.648953) (size 0.6) (drill 0.3) (layers "F.Cu" "B.Cu") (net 24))
 (via (at 140.168953 99.648953) (size 0.6) (drill 0.3) (layers "F.Cu" "B.Cu") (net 24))
 (arc (start 138.898953 101.754475) (mid 139.748799 106.026935) (end 142.168953 109.648953) (width 0.2) (layer "F.Cu") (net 24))
 (segment (start 147.882376 123.442376) (end 148.168953 123.728953) (width 0.2) (layer "B.Cu") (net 24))
 (arc (start 142.168953 109.648953) (mid 143.653823 117.1139) (end 147.882376 123.442376) (width 0.2) (layer "B.Cu") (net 24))
 (segment (start 144.458299 108.938299) (end 145.168953 109.648953) (width 0.2) (layer "F.Cu") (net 27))
 (via (at 145.168953 109.648953) (size 0.6) (drill 0.3) (layers "F.Cu" "B.Cu") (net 27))
 (arc (start 141.438953 101.648953) (mid 142.223655 105.593919) (end 144.458299 108.938299) (width 0.2) (layer "F.Cu") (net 27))
 (segment (start 147.615542 115.555543) (end 148.168953 116.108953) (width 0.2) (layer "B.Cu") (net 27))
 (arc (start 145.168953 109.648953) (mid 145.804801 112.845576) (end 147.615542 115.555543) (width 0.2) (layer "B.Cu") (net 27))
 (segment (start 116.918953 109.148953) (end 129.418953 109.148953) (width 0.2) (layer "F.Cu") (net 7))
 (segment (start 129.418953 109.148953) (end 129.509955 109.240665) (width 0.2) (layer "F.Cu") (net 7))
 (segment (start 129.601359 109.335758) (end 129.68752 109.428255) (width 0.2) (layer "F.Cu") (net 7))
 (segment (start 129.509955 109.240665) (end 129.601359 109.335758) (width 0.2) (layer "F.Cu") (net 7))
 (segment (start 131.318972 113.736005) (end 131.318972 120.648953) (width 0.2) (layer "F.Cu") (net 7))
 (arc (start 129.776102 109.526338) (mid 130.601536 110.639862) (end 131.227265 111.876639) (width 0.2) (layer "F.Cu") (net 7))
 (arc (start 129.68752 109.428255) (mid 129.73181 109.477295) (end 129.776102 109.526338) (width 0.2) (layer "F.Cu") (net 7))
 (arc (start 129.418953 109.148953) (mid 130.825173 111.253511) (end 131.318972 113.736005) (width 0.2) (layer "F.Cu") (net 7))
 (arc (start 131.227265 119.620715) (mid 131.66952 121.844077) (end 132.928953 123.728953) (width 0.2) (layer "F.Cu") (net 7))
 (segment (start 148.889713 112.10089) (end 148.822 112.119035) (width 0.2) (layer "F.Cu") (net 6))
 (segment (start 148.822 112.119035) (end 148.624531 112.119528) (width 0.2) (layer "F.Cu") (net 6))
 (segment (start 136.964556 117.153351) (end 132.928953 121.188953) (width 0.2) (layer "F.Cu") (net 6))
 (segment (start 148.954478 112.074062) (end 148.889713 112.10089) (width 0.2) (layer "F.Cu") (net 6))
 (segment (start 148.624531 112.119528) (end 148.276106 112.467953) (width 0.2) (layer "F.Cu") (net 6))
 (segment (start 149.015186 112.03901) (end 148.954478 112.074062) (width 0.2) (layer "F.Cu") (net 6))
 (segment (start 149.095971 111.971935) (end 149.0708 111.996333) (width 0.2) (layer "F.Cu") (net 6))
 (segment (start 151.918953 109.148953) (end 164.418953 109.148953) (width 0.2) (layer "F.Cu") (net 6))
 (segment (start 151.918953 109.148953) (end 149.095971 111.971935) (width 0.2) (layer "F.Cu") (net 6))
 (segment (start 149.0708 111.996333) (end 149.015186 112.03901) (width 0.2) (layer "F.Cu") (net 6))
 (arc (start 148.276106 112.467953) (mid 142.154339 113.685648) (end 136.964556 117.153351) (width 0.2) (layer "F.Cu") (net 6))
 (segment (start 148.12391 111.029488) (end 145.191866 111.029488) (width 0.2) (layer "F.Cu") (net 4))
 (segment (start 147.648837 110.508837) (end 148.168953 111.028953) (width 0.2) (layer "F.Cu") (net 4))
 (segment (start 148.168953 111.028953) (end 148.12391 111.029488) (width 0.2) (layer "F.Cu") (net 4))
 (arc (start 143.978953 101.648953) (mid 144.932725 106.443888) (end 147.648837 110.508837) (width 0.2) (layer "F.Cu") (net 4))
 (arc (start 145.191866 111.029488) (mid 138.555226 112.349598) (end 132.928953 116.108953) (width 0.2) (layer "F.Cu") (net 4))
 (segment (start 139.168953 108.432893) (end 139.168953 110.648953) (width 0.2) (layer "F.Cu") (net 23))
 (via (at 139.168953 110.648953) (size 0.6) (drill 0.3) (layers "F.Cu" "B.Cu") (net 23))
 (arc (start 136.358953 101.648953) (mid 138.438658 104.761451) (end 139.168953 108.432893) (width 0.2) (layer "F.Cu") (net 23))
 (segment (start 143.85 121.95) (end 148.168953 126.268953) (width 0.2) (layer "B.Cu") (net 23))
 (arc (start 139.168953 110.648953) (mid 140.385517 116.765036) (end 143.85 121.95) (width 0.2) (layer "B.Cu") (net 23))
 (segment (start 151.918953 114.148953) (end 164.418953 114.148953) (width 0.2) (layer "F.Cu") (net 31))
 (segment (start 129.418953 114.148953) (end 116.918953 114.148953) (width 0.2) (layer "F.Cu") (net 30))
 (via (at 130.593953 117.148953) (size 0.6) (drill 0.3) (layers "F.Cu" "B.Cu") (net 30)))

